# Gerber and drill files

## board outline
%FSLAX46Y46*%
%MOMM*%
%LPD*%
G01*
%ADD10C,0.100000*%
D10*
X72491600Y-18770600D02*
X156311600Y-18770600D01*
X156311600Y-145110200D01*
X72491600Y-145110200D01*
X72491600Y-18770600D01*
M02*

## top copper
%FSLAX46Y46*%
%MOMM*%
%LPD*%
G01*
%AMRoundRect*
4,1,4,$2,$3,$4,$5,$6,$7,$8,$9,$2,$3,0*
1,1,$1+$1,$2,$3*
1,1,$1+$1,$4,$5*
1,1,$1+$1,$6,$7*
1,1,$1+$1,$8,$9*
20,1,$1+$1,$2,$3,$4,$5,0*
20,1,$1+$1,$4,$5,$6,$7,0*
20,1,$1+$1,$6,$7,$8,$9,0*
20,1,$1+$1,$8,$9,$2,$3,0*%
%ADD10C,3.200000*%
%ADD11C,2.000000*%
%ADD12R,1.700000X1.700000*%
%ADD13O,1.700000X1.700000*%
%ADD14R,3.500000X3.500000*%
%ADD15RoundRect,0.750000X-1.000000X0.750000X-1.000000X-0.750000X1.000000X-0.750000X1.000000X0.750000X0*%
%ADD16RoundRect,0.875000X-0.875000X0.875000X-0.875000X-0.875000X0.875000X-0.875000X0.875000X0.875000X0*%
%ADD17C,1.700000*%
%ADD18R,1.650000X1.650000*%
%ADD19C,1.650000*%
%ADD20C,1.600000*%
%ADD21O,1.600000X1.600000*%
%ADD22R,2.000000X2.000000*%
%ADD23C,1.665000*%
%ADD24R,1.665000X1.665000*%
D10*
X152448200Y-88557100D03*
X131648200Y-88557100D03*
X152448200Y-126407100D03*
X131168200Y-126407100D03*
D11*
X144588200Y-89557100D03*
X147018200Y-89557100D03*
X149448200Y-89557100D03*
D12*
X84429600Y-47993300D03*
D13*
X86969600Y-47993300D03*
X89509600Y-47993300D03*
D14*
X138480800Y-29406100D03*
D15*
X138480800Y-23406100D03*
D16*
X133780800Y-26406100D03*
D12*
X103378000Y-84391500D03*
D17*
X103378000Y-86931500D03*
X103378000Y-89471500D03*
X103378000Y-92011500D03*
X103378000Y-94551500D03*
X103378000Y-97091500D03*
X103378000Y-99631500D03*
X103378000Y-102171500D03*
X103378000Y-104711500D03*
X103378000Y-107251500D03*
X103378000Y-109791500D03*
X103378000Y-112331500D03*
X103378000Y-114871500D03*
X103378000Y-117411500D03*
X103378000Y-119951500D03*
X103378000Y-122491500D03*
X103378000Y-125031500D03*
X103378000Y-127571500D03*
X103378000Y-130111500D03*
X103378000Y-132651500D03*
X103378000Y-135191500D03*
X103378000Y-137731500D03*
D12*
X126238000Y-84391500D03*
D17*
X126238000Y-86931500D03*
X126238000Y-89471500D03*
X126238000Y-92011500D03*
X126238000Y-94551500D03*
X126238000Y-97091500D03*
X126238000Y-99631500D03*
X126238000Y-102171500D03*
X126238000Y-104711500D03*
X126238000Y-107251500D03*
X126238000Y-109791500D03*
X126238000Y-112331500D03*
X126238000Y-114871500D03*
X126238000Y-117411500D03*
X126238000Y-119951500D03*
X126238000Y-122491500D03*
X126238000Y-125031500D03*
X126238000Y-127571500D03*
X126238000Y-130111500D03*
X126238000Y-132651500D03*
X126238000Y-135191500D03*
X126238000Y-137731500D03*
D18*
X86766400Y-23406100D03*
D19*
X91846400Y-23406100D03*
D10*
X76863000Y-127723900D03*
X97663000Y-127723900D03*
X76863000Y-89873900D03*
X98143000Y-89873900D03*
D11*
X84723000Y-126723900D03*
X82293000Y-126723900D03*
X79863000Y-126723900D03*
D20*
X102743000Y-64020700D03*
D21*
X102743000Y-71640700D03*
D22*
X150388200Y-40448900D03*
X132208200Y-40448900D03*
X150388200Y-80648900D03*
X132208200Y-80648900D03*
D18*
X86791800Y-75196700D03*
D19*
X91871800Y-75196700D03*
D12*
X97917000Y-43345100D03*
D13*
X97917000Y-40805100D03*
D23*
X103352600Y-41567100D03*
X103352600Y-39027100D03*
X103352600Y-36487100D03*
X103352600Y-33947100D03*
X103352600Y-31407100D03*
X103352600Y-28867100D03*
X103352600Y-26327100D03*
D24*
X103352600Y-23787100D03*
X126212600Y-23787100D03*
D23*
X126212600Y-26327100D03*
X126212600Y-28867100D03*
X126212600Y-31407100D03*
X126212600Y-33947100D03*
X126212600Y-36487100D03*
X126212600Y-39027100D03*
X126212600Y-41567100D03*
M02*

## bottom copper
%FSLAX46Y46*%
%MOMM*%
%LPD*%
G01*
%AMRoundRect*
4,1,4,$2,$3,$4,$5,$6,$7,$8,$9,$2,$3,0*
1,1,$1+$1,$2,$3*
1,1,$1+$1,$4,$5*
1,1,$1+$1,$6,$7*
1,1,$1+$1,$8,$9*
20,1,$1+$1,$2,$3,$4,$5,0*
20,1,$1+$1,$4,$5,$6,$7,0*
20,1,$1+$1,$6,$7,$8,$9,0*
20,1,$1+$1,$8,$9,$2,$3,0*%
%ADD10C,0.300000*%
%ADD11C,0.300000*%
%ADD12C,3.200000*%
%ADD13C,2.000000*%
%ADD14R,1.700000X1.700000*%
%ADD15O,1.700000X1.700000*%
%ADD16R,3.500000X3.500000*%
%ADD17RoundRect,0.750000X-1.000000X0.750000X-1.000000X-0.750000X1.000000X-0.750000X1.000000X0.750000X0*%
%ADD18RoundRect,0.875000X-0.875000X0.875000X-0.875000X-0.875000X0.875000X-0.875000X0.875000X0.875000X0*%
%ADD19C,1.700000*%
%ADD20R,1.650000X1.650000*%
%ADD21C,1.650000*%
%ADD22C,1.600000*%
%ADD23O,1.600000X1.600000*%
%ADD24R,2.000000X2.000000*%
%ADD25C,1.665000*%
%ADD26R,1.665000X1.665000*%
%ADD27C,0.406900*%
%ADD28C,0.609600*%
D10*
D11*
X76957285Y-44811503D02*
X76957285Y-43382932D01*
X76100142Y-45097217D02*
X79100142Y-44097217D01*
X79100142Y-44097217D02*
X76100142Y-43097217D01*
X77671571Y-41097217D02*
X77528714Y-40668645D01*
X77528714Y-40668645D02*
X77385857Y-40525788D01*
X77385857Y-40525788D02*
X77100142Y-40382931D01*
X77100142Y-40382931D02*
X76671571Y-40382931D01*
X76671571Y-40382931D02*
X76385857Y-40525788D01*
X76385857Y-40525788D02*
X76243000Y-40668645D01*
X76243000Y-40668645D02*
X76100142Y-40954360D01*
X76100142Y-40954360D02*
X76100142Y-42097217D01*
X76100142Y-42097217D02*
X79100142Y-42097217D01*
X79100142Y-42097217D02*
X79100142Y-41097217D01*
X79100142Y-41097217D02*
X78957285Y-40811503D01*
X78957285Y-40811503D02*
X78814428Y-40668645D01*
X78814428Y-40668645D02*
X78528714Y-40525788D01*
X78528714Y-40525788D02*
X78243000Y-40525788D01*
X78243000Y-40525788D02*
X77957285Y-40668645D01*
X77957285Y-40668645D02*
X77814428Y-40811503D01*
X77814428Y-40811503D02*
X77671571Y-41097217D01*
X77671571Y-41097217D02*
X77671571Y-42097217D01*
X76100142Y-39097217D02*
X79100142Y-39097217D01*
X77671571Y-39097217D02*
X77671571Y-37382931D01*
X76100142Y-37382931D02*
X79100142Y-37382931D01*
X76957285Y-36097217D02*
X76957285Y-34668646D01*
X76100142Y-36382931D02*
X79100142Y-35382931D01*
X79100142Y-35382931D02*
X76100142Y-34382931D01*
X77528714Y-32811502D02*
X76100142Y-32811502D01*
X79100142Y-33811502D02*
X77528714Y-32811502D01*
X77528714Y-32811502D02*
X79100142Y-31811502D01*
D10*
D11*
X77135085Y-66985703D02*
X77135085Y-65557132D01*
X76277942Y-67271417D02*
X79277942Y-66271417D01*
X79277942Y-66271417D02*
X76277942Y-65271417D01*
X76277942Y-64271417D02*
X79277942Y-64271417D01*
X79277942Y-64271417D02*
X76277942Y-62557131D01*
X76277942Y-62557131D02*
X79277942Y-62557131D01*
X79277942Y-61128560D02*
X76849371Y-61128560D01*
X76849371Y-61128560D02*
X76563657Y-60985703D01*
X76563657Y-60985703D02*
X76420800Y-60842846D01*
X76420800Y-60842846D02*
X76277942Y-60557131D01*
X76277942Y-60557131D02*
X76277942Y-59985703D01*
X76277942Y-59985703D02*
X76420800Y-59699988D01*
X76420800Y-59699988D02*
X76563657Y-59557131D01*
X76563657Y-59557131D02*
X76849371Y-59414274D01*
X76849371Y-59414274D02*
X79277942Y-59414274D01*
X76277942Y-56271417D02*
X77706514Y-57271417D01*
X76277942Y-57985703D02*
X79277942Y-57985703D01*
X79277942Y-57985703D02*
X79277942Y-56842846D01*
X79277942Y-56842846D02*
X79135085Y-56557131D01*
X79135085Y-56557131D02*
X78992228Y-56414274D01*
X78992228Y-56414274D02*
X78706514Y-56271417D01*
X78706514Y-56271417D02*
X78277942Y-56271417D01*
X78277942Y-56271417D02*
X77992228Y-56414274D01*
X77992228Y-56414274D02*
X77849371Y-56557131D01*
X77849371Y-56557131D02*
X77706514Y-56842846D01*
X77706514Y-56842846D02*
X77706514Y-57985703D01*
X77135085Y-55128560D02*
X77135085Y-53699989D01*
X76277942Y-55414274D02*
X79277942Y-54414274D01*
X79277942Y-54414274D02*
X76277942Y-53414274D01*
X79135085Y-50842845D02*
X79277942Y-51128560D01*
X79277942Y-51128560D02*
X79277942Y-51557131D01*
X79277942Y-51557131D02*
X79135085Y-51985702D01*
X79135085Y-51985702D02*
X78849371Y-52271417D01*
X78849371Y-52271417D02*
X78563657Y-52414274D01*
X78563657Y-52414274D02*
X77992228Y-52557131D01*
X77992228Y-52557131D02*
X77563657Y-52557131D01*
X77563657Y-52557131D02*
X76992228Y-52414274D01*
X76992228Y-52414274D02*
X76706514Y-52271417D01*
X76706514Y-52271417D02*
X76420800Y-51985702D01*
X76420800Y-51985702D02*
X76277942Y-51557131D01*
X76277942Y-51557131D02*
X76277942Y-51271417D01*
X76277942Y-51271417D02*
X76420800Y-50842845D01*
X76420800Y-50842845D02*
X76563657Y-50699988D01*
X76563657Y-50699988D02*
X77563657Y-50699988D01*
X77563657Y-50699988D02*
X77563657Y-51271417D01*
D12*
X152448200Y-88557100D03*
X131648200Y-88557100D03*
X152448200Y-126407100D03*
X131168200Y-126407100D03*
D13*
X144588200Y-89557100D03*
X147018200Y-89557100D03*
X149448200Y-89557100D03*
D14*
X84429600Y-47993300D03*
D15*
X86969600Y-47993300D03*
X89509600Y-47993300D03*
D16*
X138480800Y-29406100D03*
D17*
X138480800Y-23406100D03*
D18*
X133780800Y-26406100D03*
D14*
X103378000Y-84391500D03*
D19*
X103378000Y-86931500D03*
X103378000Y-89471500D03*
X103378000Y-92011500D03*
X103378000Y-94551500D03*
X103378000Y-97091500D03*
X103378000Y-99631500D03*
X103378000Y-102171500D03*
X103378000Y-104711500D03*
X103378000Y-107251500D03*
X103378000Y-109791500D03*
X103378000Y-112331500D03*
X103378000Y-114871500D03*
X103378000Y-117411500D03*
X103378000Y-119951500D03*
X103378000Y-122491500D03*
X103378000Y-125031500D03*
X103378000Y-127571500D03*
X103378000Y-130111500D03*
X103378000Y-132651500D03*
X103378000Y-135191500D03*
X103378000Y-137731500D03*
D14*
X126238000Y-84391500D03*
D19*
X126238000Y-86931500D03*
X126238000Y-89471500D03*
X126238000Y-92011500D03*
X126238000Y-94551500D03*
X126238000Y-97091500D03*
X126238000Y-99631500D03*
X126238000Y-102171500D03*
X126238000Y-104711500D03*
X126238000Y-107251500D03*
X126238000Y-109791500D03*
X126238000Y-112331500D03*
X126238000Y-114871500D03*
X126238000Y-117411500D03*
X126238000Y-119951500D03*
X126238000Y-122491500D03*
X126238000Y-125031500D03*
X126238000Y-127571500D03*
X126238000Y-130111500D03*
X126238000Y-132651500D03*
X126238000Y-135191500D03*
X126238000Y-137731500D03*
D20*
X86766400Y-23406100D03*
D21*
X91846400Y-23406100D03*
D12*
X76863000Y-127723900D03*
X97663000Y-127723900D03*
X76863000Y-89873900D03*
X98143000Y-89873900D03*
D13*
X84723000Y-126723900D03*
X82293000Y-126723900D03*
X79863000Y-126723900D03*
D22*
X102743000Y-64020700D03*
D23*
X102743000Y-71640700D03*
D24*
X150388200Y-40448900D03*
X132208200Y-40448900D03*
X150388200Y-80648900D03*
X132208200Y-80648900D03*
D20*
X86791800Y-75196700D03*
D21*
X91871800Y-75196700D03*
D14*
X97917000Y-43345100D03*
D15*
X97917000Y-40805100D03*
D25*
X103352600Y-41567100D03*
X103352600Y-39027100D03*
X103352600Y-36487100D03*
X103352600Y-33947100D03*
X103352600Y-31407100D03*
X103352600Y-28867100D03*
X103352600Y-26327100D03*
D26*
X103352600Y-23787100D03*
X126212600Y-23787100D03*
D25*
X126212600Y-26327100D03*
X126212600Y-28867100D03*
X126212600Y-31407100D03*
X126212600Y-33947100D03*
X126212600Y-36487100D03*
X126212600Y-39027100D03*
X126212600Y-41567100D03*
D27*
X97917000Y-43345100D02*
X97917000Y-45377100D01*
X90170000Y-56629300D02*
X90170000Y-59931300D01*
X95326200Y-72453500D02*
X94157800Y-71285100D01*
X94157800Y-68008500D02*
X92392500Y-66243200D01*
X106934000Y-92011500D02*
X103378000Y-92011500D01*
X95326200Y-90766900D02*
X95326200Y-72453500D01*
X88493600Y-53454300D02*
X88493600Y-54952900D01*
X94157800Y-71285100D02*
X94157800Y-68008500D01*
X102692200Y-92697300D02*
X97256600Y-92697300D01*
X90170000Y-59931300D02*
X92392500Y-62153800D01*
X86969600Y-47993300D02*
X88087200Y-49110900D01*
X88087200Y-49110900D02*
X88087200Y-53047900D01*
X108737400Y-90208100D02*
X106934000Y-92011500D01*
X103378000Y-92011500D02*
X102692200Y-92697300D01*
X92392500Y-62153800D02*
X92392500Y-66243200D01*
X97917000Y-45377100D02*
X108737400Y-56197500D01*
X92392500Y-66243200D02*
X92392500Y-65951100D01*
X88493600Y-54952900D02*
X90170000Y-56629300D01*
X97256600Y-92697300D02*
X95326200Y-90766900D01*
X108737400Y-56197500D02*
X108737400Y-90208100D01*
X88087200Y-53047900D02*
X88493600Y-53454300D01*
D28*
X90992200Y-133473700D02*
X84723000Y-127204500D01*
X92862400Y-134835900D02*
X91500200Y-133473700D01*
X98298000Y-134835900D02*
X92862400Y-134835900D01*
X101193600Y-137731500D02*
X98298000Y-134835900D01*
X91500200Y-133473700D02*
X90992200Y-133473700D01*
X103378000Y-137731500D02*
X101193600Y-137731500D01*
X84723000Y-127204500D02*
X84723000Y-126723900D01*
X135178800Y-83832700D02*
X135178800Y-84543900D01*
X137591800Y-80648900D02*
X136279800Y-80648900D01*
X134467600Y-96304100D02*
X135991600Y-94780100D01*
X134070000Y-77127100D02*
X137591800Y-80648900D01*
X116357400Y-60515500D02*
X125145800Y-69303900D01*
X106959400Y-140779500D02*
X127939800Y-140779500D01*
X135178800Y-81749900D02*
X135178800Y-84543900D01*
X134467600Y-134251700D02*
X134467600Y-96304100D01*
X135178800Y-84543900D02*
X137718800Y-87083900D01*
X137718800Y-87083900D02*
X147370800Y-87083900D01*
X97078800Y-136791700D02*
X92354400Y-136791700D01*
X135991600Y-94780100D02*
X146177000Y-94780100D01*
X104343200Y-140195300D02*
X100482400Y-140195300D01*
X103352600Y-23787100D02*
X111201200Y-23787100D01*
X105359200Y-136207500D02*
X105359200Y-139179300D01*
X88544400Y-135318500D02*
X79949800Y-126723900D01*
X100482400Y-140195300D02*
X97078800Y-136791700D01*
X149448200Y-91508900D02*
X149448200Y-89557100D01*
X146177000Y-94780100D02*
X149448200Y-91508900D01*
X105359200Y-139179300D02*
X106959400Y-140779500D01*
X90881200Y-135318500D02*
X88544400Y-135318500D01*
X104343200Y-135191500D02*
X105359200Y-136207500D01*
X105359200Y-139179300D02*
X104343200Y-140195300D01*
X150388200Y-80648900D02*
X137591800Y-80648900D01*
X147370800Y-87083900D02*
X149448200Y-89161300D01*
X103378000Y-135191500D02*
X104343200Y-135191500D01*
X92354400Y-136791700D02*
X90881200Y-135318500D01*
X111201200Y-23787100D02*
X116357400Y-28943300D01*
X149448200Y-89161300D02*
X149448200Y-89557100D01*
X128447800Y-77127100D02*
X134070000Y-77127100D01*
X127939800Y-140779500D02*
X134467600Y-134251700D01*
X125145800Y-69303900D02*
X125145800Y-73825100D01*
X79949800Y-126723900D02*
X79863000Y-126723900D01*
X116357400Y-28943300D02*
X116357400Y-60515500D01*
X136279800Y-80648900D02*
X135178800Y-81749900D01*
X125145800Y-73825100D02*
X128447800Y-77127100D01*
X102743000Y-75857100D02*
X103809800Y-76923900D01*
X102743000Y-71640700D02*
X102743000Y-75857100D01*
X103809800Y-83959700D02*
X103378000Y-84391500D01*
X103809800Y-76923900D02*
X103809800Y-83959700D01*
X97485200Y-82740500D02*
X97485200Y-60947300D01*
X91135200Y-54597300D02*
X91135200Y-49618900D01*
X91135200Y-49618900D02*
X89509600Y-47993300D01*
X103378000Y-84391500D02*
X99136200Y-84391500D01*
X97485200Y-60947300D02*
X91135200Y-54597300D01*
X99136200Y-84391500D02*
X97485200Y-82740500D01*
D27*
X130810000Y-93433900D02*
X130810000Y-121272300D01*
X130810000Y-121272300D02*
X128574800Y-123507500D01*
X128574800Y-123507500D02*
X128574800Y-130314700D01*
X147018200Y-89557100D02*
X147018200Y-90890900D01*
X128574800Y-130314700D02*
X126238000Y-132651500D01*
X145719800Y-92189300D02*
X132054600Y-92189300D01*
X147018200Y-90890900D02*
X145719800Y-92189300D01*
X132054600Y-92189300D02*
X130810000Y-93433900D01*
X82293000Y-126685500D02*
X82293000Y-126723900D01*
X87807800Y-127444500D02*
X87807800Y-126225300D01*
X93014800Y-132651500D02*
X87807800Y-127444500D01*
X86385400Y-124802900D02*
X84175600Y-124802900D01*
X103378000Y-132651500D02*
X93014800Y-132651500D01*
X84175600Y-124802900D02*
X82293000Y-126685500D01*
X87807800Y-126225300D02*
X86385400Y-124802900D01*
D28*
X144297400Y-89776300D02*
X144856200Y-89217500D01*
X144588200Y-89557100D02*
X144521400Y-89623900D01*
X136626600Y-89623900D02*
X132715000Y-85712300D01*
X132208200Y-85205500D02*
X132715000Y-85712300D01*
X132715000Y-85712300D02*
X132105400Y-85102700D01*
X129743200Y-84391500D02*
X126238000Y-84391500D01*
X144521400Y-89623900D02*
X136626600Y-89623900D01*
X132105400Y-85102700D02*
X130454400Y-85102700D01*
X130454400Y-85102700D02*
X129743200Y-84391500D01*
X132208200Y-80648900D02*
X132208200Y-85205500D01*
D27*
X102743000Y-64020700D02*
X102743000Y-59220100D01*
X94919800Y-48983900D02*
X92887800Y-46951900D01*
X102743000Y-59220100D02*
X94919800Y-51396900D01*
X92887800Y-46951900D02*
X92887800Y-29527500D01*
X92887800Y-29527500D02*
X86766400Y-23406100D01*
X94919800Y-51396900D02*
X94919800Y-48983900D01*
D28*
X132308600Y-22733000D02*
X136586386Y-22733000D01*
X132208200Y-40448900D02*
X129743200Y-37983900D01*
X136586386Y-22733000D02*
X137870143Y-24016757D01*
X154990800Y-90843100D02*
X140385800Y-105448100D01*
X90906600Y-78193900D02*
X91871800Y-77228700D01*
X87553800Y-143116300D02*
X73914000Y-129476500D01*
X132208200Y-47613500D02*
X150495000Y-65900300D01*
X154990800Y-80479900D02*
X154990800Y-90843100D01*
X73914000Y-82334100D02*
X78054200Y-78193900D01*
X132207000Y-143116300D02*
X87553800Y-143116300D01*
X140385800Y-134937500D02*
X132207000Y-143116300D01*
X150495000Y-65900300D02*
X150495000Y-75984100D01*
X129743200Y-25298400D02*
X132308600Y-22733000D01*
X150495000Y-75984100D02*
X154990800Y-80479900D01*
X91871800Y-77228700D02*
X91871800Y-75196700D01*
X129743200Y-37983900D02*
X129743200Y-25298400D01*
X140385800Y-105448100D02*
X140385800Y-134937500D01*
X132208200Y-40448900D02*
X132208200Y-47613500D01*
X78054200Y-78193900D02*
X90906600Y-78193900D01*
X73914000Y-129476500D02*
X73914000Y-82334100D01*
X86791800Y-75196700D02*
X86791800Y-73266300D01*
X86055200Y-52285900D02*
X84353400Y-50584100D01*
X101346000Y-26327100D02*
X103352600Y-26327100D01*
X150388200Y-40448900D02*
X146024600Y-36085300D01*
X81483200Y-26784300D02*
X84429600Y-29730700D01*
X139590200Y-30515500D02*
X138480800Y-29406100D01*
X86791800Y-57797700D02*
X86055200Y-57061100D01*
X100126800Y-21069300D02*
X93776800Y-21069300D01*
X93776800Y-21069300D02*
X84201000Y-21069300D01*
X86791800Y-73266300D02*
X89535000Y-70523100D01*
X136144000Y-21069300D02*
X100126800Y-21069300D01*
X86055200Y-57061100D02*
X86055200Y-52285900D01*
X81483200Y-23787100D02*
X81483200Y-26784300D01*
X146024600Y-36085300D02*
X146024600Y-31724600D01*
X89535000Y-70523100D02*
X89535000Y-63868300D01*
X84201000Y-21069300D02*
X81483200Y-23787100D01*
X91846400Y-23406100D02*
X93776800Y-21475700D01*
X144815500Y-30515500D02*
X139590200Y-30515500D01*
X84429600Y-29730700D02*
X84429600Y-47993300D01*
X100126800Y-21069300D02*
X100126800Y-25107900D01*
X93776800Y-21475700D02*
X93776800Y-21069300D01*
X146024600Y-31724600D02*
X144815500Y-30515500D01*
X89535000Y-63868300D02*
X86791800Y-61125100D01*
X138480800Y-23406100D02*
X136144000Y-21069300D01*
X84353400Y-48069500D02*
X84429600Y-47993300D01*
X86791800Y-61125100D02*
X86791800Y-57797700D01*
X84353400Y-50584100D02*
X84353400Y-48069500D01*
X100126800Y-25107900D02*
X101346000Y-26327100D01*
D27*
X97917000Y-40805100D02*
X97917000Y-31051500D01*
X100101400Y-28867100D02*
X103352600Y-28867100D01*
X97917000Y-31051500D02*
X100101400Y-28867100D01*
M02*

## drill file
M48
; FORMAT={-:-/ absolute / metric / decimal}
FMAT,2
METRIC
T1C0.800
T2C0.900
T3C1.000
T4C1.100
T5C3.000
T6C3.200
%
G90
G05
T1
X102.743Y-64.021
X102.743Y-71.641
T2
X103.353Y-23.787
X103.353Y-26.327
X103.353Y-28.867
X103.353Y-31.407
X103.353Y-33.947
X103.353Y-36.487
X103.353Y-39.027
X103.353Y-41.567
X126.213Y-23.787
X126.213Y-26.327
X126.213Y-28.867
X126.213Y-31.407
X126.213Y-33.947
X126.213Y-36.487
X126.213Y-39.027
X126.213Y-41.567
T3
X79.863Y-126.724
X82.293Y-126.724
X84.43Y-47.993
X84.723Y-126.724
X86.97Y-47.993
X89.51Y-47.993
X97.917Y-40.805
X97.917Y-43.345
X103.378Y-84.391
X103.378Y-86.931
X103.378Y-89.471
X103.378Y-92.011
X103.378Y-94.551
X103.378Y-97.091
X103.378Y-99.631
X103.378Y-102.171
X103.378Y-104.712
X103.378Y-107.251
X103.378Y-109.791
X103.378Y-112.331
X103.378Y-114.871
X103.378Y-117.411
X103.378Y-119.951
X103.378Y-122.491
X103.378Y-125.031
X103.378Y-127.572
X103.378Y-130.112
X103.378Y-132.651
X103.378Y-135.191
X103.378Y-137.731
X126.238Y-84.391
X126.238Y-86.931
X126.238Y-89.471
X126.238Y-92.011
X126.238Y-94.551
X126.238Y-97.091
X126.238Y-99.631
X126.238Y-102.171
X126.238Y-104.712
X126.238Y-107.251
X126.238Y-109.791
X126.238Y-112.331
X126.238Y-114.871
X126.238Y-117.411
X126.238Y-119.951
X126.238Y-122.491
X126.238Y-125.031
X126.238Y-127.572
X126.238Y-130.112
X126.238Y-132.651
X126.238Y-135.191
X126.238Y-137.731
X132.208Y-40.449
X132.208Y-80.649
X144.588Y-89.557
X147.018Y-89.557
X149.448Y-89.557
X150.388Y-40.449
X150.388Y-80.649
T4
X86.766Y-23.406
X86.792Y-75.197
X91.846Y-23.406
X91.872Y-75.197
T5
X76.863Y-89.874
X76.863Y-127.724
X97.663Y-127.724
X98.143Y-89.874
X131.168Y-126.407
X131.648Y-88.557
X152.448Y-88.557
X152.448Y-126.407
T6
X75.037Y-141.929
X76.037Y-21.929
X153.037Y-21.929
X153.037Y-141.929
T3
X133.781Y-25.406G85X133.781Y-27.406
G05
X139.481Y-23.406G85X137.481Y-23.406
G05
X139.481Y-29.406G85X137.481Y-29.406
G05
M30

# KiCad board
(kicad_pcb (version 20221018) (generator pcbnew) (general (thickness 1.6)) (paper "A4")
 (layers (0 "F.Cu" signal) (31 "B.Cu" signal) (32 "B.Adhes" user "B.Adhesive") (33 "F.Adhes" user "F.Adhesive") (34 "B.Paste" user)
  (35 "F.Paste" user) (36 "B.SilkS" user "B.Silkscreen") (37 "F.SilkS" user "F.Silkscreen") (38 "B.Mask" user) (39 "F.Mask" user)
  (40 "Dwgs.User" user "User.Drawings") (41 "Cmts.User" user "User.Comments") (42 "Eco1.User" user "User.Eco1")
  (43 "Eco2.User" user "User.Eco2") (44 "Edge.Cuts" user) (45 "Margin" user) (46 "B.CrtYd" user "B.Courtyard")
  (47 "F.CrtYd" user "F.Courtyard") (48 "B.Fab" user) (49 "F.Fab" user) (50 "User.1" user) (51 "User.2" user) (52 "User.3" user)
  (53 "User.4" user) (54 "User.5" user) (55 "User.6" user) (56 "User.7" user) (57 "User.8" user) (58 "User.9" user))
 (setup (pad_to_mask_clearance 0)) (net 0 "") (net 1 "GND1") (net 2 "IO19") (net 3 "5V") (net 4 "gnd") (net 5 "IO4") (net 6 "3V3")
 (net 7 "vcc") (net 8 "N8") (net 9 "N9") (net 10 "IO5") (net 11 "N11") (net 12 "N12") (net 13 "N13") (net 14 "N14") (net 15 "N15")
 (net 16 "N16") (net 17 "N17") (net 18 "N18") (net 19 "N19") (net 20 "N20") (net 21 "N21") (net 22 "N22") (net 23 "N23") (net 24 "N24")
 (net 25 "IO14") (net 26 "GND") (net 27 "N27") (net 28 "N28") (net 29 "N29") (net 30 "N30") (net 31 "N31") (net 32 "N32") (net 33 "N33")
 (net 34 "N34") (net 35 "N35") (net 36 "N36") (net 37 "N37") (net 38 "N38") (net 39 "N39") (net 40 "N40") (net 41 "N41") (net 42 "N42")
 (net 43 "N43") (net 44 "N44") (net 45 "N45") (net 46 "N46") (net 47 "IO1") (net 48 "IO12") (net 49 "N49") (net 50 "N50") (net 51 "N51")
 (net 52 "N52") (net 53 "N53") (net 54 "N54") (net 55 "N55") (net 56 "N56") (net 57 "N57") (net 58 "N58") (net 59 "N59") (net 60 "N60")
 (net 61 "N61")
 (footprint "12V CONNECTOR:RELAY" (layer "F.Cu") (at 131.6482 88.5571 -90)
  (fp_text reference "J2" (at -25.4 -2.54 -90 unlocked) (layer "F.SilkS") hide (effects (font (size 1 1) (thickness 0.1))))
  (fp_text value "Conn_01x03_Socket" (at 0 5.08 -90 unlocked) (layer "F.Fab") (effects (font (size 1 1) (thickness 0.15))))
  (pad "" np_thru_hole circle (at 0 -20.8 270) (size 3.2 3.2) (drill 3) (layers "F&B.Cu" "*.Mask"))
  (pad "" np_thru_hole circle (at 0 0 270) (size 3.2 3.2) (drill 3) (layers "F&B.Cu" "*.Mask"))
  (pad "" np_thru_hole circle (at 37.85 -20.8 270) (size 3.2 3.2) (drill 3) (layers "F&B.Cu" "*.Mask"))
  (pad "" np_thru_hole circle (at 37.85 0.48 270) (size 3.2 3.2) (drill 3) (layers "F&B.Cu" "*.Mask"))
  (pad "1" thru_hole circle (at 1 -12.94 270) (size 2 2) (drill 1) (layers "*.Cu" "*.Mask") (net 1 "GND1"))
  (pad "2" thru_hole circle (at 1 -15.37 270) (size 2 2) (drill 1) (layers "*.Cu" "*.Mask") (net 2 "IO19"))
  (pad "3" thru_hole circle (at 1 -17.8 270) (size 2 2) (drill 1) (layers "*.Cu" "*.Mask") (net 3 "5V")))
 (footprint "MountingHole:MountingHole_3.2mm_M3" (layer "F.Cu") (at 153.0368 21.9289)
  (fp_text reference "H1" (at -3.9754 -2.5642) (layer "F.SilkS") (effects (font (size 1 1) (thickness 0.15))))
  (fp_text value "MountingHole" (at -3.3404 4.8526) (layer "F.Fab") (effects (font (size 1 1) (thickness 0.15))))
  (pad "" np_thru_hole circle (at 0 0) (size 3.2 3.2) (drill 3.2) (layers "*.Cu" "*.Mask")))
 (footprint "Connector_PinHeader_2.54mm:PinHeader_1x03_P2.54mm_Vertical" (layer "F.Cu") (at 84.4296 47.9933 90)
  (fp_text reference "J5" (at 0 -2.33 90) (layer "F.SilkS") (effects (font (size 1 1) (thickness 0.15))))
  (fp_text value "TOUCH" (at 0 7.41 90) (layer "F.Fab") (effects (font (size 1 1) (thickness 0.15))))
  (pad "1" thru_hole rect (at 0 0 90) (size 1.7 1.7) (drill 1) (layers "*.Cu" "*.Mask") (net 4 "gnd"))
  (pad "2" thru_hole oval (at 0 2.54 90) (size 1.7 1.7) (drill 1) (layers "*.Cu" "*.Mask") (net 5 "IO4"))
  (pad "3" thru_hole oval (at 0 5.08 90) (size 1.7 1.7) (drill 1) (layers "*.Cu" "*.Mask") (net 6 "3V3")))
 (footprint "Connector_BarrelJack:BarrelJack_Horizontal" (layer "F.Cu") (at 138.4808 29.4061 -90)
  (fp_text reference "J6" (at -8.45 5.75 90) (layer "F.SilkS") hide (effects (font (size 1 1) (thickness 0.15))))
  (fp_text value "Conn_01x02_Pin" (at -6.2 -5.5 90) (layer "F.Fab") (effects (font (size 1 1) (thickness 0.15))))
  (pad "1" thru_hole rect (at 0 0 270) (size 3.5 3.5) (drill oval 1 3) (layers "*.Cu" "*.Mask") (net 4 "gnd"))
  (pad "2" thru_hole roundrect (at -6 0 270) (size 3 3.5) (drill oval 1 3) (layers "*.Cu" "*.Mask") (roundrect_rratio 0.25) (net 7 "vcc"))
  (pad "3" thru_hole roundrect (at -3 4.7 270) (size 3.5 3.5) (drill oval 3 1) (layers "*.Cu" "*.Mask") (roundrect_rratio 0.25)))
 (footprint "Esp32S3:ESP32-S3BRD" (layer "F.Cu") (at 102.108 149.1915)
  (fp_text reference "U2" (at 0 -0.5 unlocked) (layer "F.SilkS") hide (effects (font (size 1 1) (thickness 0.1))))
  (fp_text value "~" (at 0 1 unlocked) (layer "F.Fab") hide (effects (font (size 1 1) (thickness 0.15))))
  (pad "1_1" thru_hole rect (at 1.27 -64.8) (size 1.7 1.7) (drill 1) (layers "*.Cu" "*.Mask") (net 6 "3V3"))
  (pad "1_2" thru_hole circle (at 1.27 -62.26) (size 1.7 1.7) (drill 1) (layers "*.Cu" "*.Mask") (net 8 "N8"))
  (pad "1_3" thru_hole circle (at 1.27 -59.72) (size 1.7 1.7) (drill 1) (layers "*.Cu" "*.Mask") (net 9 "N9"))
  (pad "1_4" thru_hole circle (at 1.27 -57.18) (size 1.7 1.7) (drill 1) (layers "*.Cu" "*.Mask") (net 5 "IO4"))
  (pad "1_5" thru_hole circle (at 1.27 -54.64) (size 1.7 1.7) (drill 1) (layers "*.Cu" "*.Mask") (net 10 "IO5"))
  (pad "1_6" thru_hole circle (at 1.27 -52.1) (size 1.7 1.7) (drill 1) (layers "*.Cu" "*.Mask") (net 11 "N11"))
  (pad "1_7" thru_hole circle (at 1.27 -49.56) (size 1.7 1.7) (drill 1) (layers "*.Cu" "*.Mask") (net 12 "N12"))
  (pad "1_8" thru_hole circle (at 1.27 -47.02) (size 1.7 1.7) (drill 1) (layers "*.Cu" "*.Mask") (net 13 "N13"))
  (pad "1_9" thru_hole circle (at 1.27 -44.48) (size 1.7 1.7) (drill 1) (layers "*.Cu" "*.Mask") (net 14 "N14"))
  (pad "1_10" thru_hole circle (at 1.27 -41.94) (size 1.7 1.7) (drill 1) (layers "*.Cu" "*.Mask") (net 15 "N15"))
  (pad "1_11" thru_hole circle (at 1.27 -39.4) (size 1.7 1.7) (drill 1) (layers "*.Cu" "*.Mask") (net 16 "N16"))
  (pad "1_12" thru_hole circle (at 1.27 -36.86) (size 1.7 1.7) (drill 1) (layers "*.Cu" "*.Mask") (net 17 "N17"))
  (pad "1_13" thru_hole circle (at 1.27 -34.32) (size 1.7 1.7) (drill 1) (layers "*.Cu" "*.Mask") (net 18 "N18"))
  (pad "1_14" thru_hole circle (at 1.27 -31.78) (size 1.7 1.7) (drill 1) (layers "*.Cu" "*.Mask") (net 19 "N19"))
  (pad "1_15" thru_hole circle (at 1.27 -29.24) (size 1.7 1.7) (drill 1) (layers "*.Cu" "*.Mask") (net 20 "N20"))
  (pad "1_16" thru_hole circle (at 1.27 -26.7) (size 1.7 1.7) (drill 1) (layers "*.Cu" "*.Mask") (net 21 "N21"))
  (pad "1_17" thru_hole circle (at 1.27 -24.16) (size 1.7 1.7) (drill 1) (layers "*.Cu" "*.Mask") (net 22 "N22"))
  (pad "1_18" thru_hole circle (at 1.27 -21.62) (size 1.7 1.7) (drill 1) (layers "*.Cu" "*.Mask") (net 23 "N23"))
  (pad "1_19" thru_hole circle (at 1.27 -19.08) (size 1.7 1.7) (drill 1) (layers "*.Cu" "*.Mask") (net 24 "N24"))
  (pad "1_20" thru_hole circle (at 1.27 -16.54) (size 1.7 1.7) (drill 1) (layers "*.Cu" "*.Mask") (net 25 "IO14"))
  (pad "1_21" thru_hole circle (at 1.27 -14) (size 1.7 1.7) (drill 1) (layers "*.Cu" "*.Mask") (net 3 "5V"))
  (pad "1_22" thru_hole circle (at 1.27 -11.46) (size 1.7 1.7) (drill 1) (layers "*.Cu" "*.Mask") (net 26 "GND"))
  (pad "2_1" thru_hole rect (at 24.13 -64.8) (size 1.7 1.7) (drill 1) (layers "*.Cu" "*.Mask") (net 1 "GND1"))
  (pad "2_2" thru_hole circle (at 24.13 -62.26) (size 1.7 1.7) (drill 1) (layers "*.Cu" "*.Mask") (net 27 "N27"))
  (pad "2_3" thru_hole circle (at 24.13 -59.72) (size 1.7 1.7) (drill 1) (layers "*.Cu" "*.Mask") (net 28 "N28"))
  (pad "2_4" thru_hole circle (at 24.13 -57.18) (size 1.7 1.7) (drill 1) (layers "*.Cu" "*.Mask") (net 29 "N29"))
  (pad "2_5" thru_hole circle (at 24.13 -54.64) (size 1.7 1.7) (drill 1) (layers "*.Cu" "*.Mask") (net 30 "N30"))
  (pad "2_6" thru_hole circle (at 24.13 -52.1) (size 1.7 1.7) (drill 1) (layers "*.Cu" "*.Mask") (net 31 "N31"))
  (pad "2_7" thru_hole circle (at 24.13 -49.56) (size 1.7 1.7) (drill 1) (layers "*.Cu" "*.Mask") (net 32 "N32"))
  (pad "2_8" thru_hole circle (at 24.13 -47.02) (size 1.7 1.7) (drill 1) (layers "*.Cu" "*.Mask") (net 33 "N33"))
  (pad "2_9" thru_hole circle (at 24.13 -44.48) (size 1.7 1.7) (drill 1) (layers "*.Cu" "*.Mask") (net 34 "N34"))
  (pad "2_10" thru_hole circle (at 24.13 -41.94) (size 1.7 1.7) (drill 1) (layers "*.Cu" "*.Mask") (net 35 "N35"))
  (pad "2_11" thru_hole circle (at 24.13 -39.4) (size 1.7 1.7) (drill 1) (layers "*.Cu" "*.Mask") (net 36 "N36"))
  (pad "2_12" thru_hole circle (at 24.13 -36.86) (size 1.7 1.7) (drill 1) (layers "*.Cu" "*.Mask") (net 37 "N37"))
  (pad "2_13" thru_hole circle (at 24.13 -34.32) (size 1.7 1.7) (drill 1) (layers "*.Cu" "*.Mask") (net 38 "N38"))
  (pad "2_14" thru_hole circle (at 24.13 -31.78) (size 1.7 1.7) (drill 1) (layers "*.Cu" "*.Mask") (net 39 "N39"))
  (pad "2_15" thru_hole circle (at 24.13 -29.24) (size 1.7 1.7) (drill 1) (layers "*.Cu" "*.Mask") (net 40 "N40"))
  (pad "2_16" thru_hole circle (at 24.13 -26.7) (size 1.7 1.7) (drill 1) (layers "*.Cu" "*.Mask") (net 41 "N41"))
  (pad "2_17" thru_hole circle (at 24.13 -24.16) (size 1.7 1.7) (drill 1) (layers "*.Cu" "*.Mask") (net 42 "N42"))
  (pad "2_18" thru_hole circle (at 24.13 -21.62) (size 1.7 1.7) (drill 1) (layers "*.Cu" "*.Mask") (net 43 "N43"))
  (pad "2_19" thru_hole circle (at 24.13 -19.08) (size 1.7 1.7) (drill 1) (layers "*.Cu" "*.Mask") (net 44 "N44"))
  (pad "2_20" thru_hole circle (at 24.13 -16.54) (size 1.7 1.7) (drill 1) (layers "*.Cu" "*.Mask") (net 2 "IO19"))
  (pad "2_21" thru_hole circle (at 24.13 -14) (size 1.7 1.7) (drill 1) (layers "*.Cu" "*.Mask") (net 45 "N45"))
  (pad "2_22" thru_hole circle (at 24.13 -11.46) (size 1.7 1.7) (drill 1) (layers "*.Cu" "*.Mask") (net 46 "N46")))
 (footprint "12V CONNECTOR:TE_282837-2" (layer "F.Cu") (at 89.3064 23.4061)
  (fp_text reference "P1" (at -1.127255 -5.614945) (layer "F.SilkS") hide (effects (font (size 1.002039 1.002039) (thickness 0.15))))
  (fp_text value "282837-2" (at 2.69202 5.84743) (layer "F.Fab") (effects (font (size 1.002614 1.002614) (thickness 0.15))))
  (pad "1" thru_hole rect (at -2.54 0) (size 1.65 1.65) (drill 1.1) (layers "*.Cu" "*.Mask") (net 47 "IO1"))
  (pad "2" thru_hole circle (at 2.54 0) (size 1.65 1.65) (drill 1.1) (layers "*.Cu" "*.Mask") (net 4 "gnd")))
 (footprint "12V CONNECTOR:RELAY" (layer "F.Cu") (at 97.663 127.7239 90)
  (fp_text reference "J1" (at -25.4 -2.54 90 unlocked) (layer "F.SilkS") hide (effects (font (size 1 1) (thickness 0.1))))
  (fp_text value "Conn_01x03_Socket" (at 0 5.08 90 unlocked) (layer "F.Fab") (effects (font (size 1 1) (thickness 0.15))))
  (pad "" np_thru_hole circle (at 0 -20.8 90) (size 3.2 3.2) (drill 3) (layers "F&B.Cu" "*.Mask"))
  (pad "" np_thru_hole circle (at 0 0 90) (size 3.2 3.2) (drill 3) (layers "F&B.Cu" "*.Mask"))
  (pad "" np_thru_hole circle (at 37.85 -20.8 90) (size 3.2 3.2) (drill 3) (layers "F&B.Cu" "*.Mask"))
  (pad "" np_thru_hole circle (at 37.85 0.48 90) (size 3.2 3.2) (drill 3) (layers "F&B.Cu" "*.Mask"))
  (pad "1" thru_hole circle (at 1 -12.94 90) (size 2 2) (drill 1) (layers "*.Cu" "*.Mask") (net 26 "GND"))
  (pad "2" thru_hole circle (at 1 -15.37 90) (size 2 2) (drill 1) (layers "*.Cu" "*.Mask") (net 25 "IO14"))
  (pad "3" thru_hole circle (at 1 -17.8 90) (size 2 2) (drill 1) (layers "*.Cu" "*.Mask") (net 3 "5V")))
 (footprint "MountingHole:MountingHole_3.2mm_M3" (layer "F.Cu") (at 153.0368 141.9289)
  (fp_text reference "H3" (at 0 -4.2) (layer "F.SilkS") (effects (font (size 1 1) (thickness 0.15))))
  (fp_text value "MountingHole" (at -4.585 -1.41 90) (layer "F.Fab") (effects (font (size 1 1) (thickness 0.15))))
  (pad "" np_thru_hole circle (at 0 0) (size 3.2 3.2) (drill 3.2) (layers "*.Cu" "*.Mask")))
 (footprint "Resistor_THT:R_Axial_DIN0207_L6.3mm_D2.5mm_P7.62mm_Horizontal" (layer "F.Cu") (at 102.743 64.0207 -90)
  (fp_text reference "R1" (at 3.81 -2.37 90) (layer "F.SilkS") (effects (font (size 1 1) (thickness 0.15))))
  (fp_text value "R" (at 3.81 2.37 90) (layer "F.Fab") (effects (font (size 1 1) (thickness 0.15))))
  (pad "1" thru_hole circle (at 0 0 270) (size 1.6 1.6) (drill 0.8) (layers "*.Cu" "*.Mask") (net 47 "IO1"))
  (pad "2" thru_hole oval (at 7.62 0 270) (size 1.6 1.6) (drill 0.8) (layers "*.Cu" "*.Mask") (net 6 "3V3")))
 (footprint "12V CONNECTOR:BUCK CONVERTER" (layer "F.Cu") (at 130.4082 38.6489 -90)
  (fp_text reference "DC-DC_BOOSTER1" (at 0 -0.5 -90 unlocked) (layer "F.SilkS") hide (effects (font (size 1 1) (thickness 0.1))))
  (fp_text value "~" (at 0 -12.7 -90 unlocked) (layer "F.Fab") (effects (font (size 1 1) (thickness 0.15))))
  (pad "IN+" thru_hole rect (at 1.8 -19.98 270) (size 2 2) (drill 1) (layers "*.Cu" "*.Mask") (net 4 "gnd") (thermal_bridge_angle 45))
  (pad "IN-" thru_hole rect (at 1.8 -1.8 270) (size 2 2) (drill 1) (layers "*.Cu" "B.Mask") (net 7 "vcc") (thermal_bridge_angle 45))
  (pad "OUT+" thru_hole rect (at 42 -19.98 270) (size 2 2) (drill 1) (layers "*.Cu" "*.Mask") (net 3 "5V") (thermal_bridge_angle 45))
  (pad "OUT-" thru_hole rect (at 42 -1.8 270) (size 2 2) (drill 1) (layers "*.Cu" "*.Mask") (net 1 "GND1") (thermal_bridge_angle 45)))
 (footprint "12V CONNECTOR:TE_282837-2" (layer "F.Cu") (at 89.3318 75.1967)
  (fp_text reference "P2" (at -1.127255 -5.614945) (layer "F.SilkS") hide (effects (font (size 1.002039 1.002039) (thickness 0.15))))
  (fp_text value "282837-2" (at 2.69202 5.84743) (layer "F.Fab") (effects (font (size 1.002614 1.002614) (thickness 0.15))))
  (pad "1" thru_hole rect (at -2.54 0) (size 1.65 1.65) (drill 1.1) (layers "*.Cu" "*.Mask") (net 4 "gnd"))
  (pad "2" thru_hole circle (at 2.54 0) (size 1.65 1.65) (drill 1.1) (layers "*.Cu" "*.Mask") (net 7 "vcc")))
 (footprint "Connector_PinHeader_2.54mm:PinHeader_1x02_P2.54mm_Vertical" (layer "F.Cu") (at 97.917 43.3451 180)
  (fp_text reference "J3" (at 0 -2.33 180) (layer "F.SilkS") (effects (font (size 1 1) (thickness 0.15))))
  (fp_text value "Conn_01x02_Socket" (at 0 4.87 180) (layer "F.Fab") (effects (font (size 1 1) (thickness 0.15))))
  (pad "1" thru_hole rect (at 0 0 180) (size 1.7 1.7) (drill 1) (layers "*.Cu" "*.Mask") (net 5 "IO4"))
  (pad "2" thru_hole oval (at 0 2.54 180) (size 1.7 1.7) (drill 1) (layers "*.Cu" "*.Mask") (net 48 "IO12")))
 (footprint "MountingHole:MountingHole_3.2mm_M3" (layer "F.Cu") (at 75.0368 141.9289)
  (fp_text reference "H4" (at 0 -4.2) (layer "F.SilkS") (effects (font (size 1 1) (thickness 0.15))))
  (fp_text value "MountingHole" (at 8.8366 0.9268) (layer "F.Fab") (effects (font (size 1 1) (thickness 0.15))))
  (pad "" np_thru_hole circle (at 0 0) (size 3.2 3.2) (drill 3.2) (layers "*.Cu" "*.Mask")))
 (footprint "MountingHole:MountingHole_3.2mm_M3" (layer "F.Cu") (at 76.0368 21.9289)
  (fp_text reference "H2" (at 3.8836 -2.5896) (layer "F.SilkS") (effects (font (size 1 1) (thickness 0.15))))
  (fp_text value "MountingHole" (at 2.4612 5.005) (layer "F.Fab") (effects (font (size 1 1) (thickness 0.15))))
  (pad "" np_thru_hole circle (at 0 0) (size 3.2 3.2) (drill 3.2) (layers "*.Cu" "*.Mask")))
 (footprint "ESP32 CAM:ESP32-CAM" (layer "F.Cu") (at 103.3526 41.5671)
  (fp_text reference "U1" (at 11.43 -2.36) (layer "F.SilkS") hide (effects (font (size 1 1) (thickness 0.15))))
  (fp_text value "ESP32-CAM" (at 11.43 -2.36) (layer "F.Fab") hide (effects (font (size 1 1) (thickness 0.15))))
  (pad "1" thru_hole circle (at 0 0) (size 1.665 1.665) (drill 0.9) (layers "*.Cu" "*.Mask") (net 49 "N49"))
  (pad "2" thru_hole circle (at 0 -2.54) (size 1.665 1.665) (drill 0.9) (layers "*.Cu" "*.Mask") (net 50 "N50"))
  (pad "3" thru_hole circle (at 0 -5.08) (size 1.665 1.665) (drill 0.9) (layers "*.Cu" "*.Mask") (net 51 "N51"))
  (pad "4" thru_hole circle (at 0 -7.62) (size 1.665 1.665) (drill 0.9) (layers "*.Cu" "*.Mask") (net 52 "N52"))
  (pad "5" thru_hole circle (at 0 -10.16) (size 1.665 1.665) (drill 0.9) (layers "*.Cu" "*.Mask") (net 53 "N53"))
  (pad "6" thru_hole circle (at 0 -12.7) (size 1.665 1.665) (drill 0.9) (layers "*.Cu" "*.Mask") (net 48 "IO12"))
  (pad "7" thru_hole circle (at 0 -15.24) (size 1.665 1.665) (drill 0.9) (layers "*.Cu" "*.Mask") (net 4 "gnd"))
  (pad "8" thru_hole rect (at 0 -17.78) (size 1.665 1.665) (drill 0.9) (layers "*.Cu" "*.Mask") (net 3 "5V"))
  (pad "9" thru_hole rect (at 22.86 -17.78) (size 1.665 1.665) (drill 0.9) (layers "*.Cu" "*.Mask") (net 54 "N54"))
  (pad "10" thru_hole circle (at 22.86 -15.24) (size 1.665 1.665) (drill 0.9) (layers "*.Cu" "*.Mask") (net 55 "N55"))
  (pad "11" thru_hole circle (at 22.86 -12.7) (size 1.665 1.665) (drill 0.9) (layers "*.Cu" "*.Mask") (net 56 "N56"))
  (pad "12" thru_hole circle (at 22.86 -10.16) (size 1.665 1.665) (drill 0.9) (layers "*.Cu" "*.Mask") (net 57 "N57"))
  (pad "13" thru_hole circle (at 22.86 -7.62) (size 1.665 1.665) (drill 0.9) (layers "*.Cu" "*.Mask") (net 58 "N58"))
  (pad "14" thru_hole circle (at 22.86 -5.08) (size 1.665 1.665) (drill 0.9) (layers "*.Cu" "*.Mask") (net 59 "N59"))
  (pad "15" thru_hole circle (at 22.86 -2.54) (size 1.665 1.665) (drill 0.9) (layers "*.Cu" "*.Mask") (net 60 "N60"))
  (pad "16" thru_hole circle (at 22.86 0) (size 1.665 1.665) (drill 0.9) (layers "*.Cu" "*.Mask") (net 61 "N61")))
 (gr_rect (start 72.4916 18.7706) (end 156.3116 145.1102) (stroke (width 0.1) (type default)) (fill none) (layer "Edge.Cuts"))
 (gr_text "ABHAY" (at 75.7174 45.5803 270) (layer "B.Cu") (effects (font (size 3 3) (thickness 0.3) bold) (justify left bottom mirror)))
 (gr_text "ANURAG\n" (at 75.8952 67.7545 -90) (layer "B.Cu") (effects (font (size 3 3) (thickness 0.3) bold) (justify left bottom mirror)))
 (segment (start 97.917 43.3451) (end 97.917 45.3771) (width 0.4069) (layer "B.Cu") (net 5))
 (segment (start 90.17 56.6293) (end 90.17 59.9313) (width 0.4069) (layer "B.Cu") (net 5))
 (segment (start 95.3262 72.4535) (end 94.1578 71.2851) (width 0.4069) (layer "B.Cu") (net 5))
 (segment (start 94.1578 68.0085) (end 92.3925 66.2432) (width 0.4069) (layer "B.Cu") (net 5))
 (segment (start 106.934 92.0115) (end 103.378 92.0115) (width 0.4069) (layer "B.Cu") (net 5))
 (segment (start 95.3262 90.7669) (end 95.3262 72.4535) (width 0.4069) (layer "B.Cu") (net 5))
 (segment (start 88.4936 53.4543) (end 88.4936 54.9529) (width 0.4069) (layer "B.Cu") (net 5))
 (segment (start 94.1578 71.2851) (end 94.1578 68.0085) (width 0.4069) (layer "B.Cu") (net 5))
 (segment (start 102.6922 92.6973) (end 97.2566 92.6973) (width 0.4069) (layer "B.Cu") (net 5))
 (segment (start 90.17 59.9313) (end 92.3925 62.1538) (width 0.4069) (layer "B.Cu") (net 5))
 (segment (start 86.9696 47.9933) (end 88.0872 49.1109) (width 0.4069) (layer "B.Cu") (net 5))
 (segment (start 88.0872 49.1109) (end 88.0872 53.0479) (width 0.4069) (layer "B.Cu") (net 5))
 (segment (start 108.7374 90.2081) (end 106.934 92.0115) (width 0.4069) (layer "B.Cu") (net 5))
 (segment (start 103.378 92.0115) (end 102.6922 92.6973) (width 0.4069) (layer "B.Cu") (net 5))
 (segment (start 92.3925 62.1538) (end 92.3925 66.2432) (width 0.4069) (layer "B.Cu") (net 5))
 (segment (start 97.917 45.3771) (end 108.7374 56.1975) (width 0.4069) (layer "B.Cu") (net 5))
 (segment (start 92.3925 66.2432) (end 92.3925 65.9511) (width 0.4069) (layer "B.Cu") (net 5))
 (segment (start 88.4936 54.9529) (end 90.17 56.6293) (width 0.4069) (layer "B.Cu") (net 5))
 (segment (start 97.2566 92.6973) (end 95.3262 90.7669) (width 0.4069) (layer "B.Cu") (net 5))
 (segment (start 108.7374 56.1975) (end 108.7374 90.2081) (width 0.4069) (layer "B.Cu") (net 5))
 (segment (start 88.0872 53.0479) (end 88.4936 53.4543) (width 0.4069) (layer "B.Cu") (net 5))
 (segment (start 90.9922 133.4737) (end 84.723 127.2045) (width 0.6096) (layer "B.Cu") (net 26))
 (segment (start 92.8624 134.8359) (end 91.5002 133.4737) (width 0.6096) (layer "B.Cu") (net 26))
 (segment (start 98.298 134.8359) (end 92.8624 134.8359) (width 0.6096) (layer "B.Cu") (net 26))
 (segment (start 101.1936 137.7315) (end 98.298 134.8359) (width 0.6096) (layer "B.Cu") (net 26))
 (segment (start 91.5002 133.4737) (end 90.9922 133.4737) (width 0.6096) (layer "B.Cu") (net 26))
 (segment (start 103.378 137.7315) (end 101.1936 137.7315) (width 0.6096) (layer "B.Cu") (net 26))
 (segment (start 84.723 127.2045) (end 84.723 126.7239) (width 0.6096) (layer "B.Cu") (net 26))
 (segment (start 135.1788 83.8327) (end 135.1788 84.5439) (width 0.6096) (layer "B.Cu") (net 3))
 (segment (start 137.5918 80.6489) (end 136.2798 80.6489) (width 0.6096) (layer "B.Cu") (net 3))
 (segment (start 134.4676 96.3041) (end 135.9916 94.7801) (width 0.6096) (layer "B.Cu") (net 3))
 (segment (start 134.07 77.1271) (end 137.5918 80.6489) (width 0.6096) (layer "B.Cu") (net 3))
 (segment (start 116.3574 60.5155) (end 125.1458 69.3039) (width 0.6096) (layer "B.Cu") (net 3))
 (segment (start 106.9594 140.7795) (end 127.9398 140.7795) (width 0.6096) (layer "B.Cu") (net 3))
 (segment (start 135.1788 81.7499) (end 135.1788 84.5439) (width 0.6096) (layer "B.Cu") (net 3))
 (segment (start 134.4676 134.2517) (end 134.4676 96.3041) (width 0.6096) (layer "B.Cu") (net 3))
 (segment (start 135.1788 84.5439) (end 137.7188 87.0839) (width 0.6096) (layer "B.Cu") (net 3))
 (segment (start 137.7188 87.0839) (end 147.3708 87.0839) (width 0.6096) (layer "B.Cu") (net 3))
 (segment (start 97.0788 136.7917) (end 92.3544 136.7917) (width 0.6096) (layer "B.Cu") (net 3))
 (segment (start 135.9916 94.7801) (end 146.177 94.7801) (width 0.6096) (layer "B.Cu") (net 3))
 (segment (start 104.3432 140.1953) (end 100.4824 140.1953) (width 0.6096) (layer "B.Cu") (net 3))
 (segment (start 103.3526 23.7871) (end 111.2012 23.7871) (width 0.6096) (layer "B.Cu") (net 3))
 (segment (start 105.3592 136.2075) (end 105.3592 139.1793) (width 0.6096) (layer "B.Cu") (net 3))
 (segment (start 88.5444 135.3185) (end 79.9498 126.7239) (width 0.6096) (layer "B.Cu") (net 3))
 (segment (start 100.4824 140.1953) (end 97.0788 136.7917) (width 0.6096) (layer "B.Cu") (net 3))
 (segment (start 149.4482 91.5089) (end 149.4482 89.5571) (width 0.6096) (layer "B.Cu") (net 3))
 (segment (start 146.177 94.7801) (end 149.4482 91.5089) (width 0.6096) (layer "B.Cu") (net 3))
 (segment (start 105.3592 139.1793) (end 106.9594 140.7795) (width 0.6096) (layer "B.Cu") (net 3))
 (segment (start 90.8812 135.3185) (end 88.5444 135.3185) (width 0.6096) (layer "B.Cu") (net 3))
 (segment (start 104.3432 135.1915) (end 105.3592 136.2075) (width 0.6096) (layer "B.Cu") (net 3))
 (segment (start 105.3592 139.1793) (end 104.3432 140.1953) (width 0.6096) (layer "B.Cu") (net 3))
 (segment (start 150.3882 80.6489) (end 137.5918 80.6489) (width 0.6096) (layer "B.Cu") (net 3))
 (segment (start 147.3708 87.0839) (end 149.4482 89.1613) (width 0.6096) (layer "B.Cu") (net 3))
 (segment (start 103.378 135.1915) (end 104.3432 135.1915) (width 0.6096) (layer "B.Cu") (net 3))
 (segment (start 92.3544 136.7917) (end 90.8812 135.3185) (width 0.6096) (layer "B.Cu") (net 3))
 (segment (start 111.2012 23.7871) (end 116.3574 28.9433) (width 0.6096) (layer "B.Cu") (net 3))
 (segment (start 149.4482 89.1613) (end 149.4482 89.5571) (width 0.6096) (layer "B.Cu") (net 3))
 (segment (start 128.4478 77.1271) (end 134.07 77.1271) (width 0.6096) (layer "B.Cu") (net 3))
 (segment (start 127.9398 140.7795) (end 134.4676 134.2517) (width 0.6096) (layer "B.Cu") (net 3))
 (segment (start 125.1458 69.3039) (end 125.1458 73.8251) (width 0.6096) (layer "B.Cu") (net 3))
 (segment (start 79.9498 126.7239) (end 79.863 126.7239) (width 0.6096) (layer "B.Cu") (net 3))
 (segment (start 116.3574 28.9433) (end 116.3574 60.5155) (width 0.6096) (layer "B.Cu") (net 3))
 (segment (start 136.2798 80.6489) (end 135.1788 81.7499) (width 0.6096) (layer "B.Cu") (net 3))
 (segment (start 125.1458 73.8251) (end 128.4478 77.1271) (width 0.6096) (layer "B.Cu") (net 3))
 (segment (start 102.743 75.8571) (end 103.8098 76.9239) (width 0.6096) (layer "B.Cu") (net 6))
 (segment (start 102.743 71.6407) (end 102.743 75.8571) (width 0.6096) (layer "B.Cu") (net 6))
 (segment (start 103.8098 83.9597) (end 103.378 84.3915) (width 0.6096) (layer "B.Cu") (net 6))
 (segment (start 103.8098 76.9239) (end 103.8098 83.9597) (width 0.6096) (layer "B.Cu") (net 6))
 (segment (start 97.4852 82.7405) (end 97.4852 60.9473) (width 0.6096) (layer "B.Cu") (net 6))
 (segment (start 91.1352 54.5973) (end 91.1352 49.6189) (width 0.6096) (layer "B.Cu") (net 6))
 (segment (start 91.1352 49.6189) (end 89.5096 47.9933) (width 0.6096) (layer "B.Cu") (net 6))
 (segment (start 103.378 84.3915) (end 99.1362 84.3915) (width 0.6096) (layer "B.Cu") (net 6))
 (segment (start 97.4852 60.9473) (end 91.1352 54.5973) (width 0.6096) (layer "B.Cu") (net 6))
 (segment (start 99.1362 84.3915) (end 97.4852 82.7405) (width 0.6096) (layer "B.Cu") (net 6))
 (segment (start 130.81 93.4339) (end 130.81 121.2723) (width 0.4069) (layer "B.Cu") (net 2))
 (segment (start 130.81 121.2723) (end 128.5748 123.5075) (width 0.4069) (layer "B.Cu") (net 2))
 (segment (start 128.5748 123.5075) (end 128.5748 130.3147) (width 0.4069) (layer "B.Cu") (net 2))
 (segment (start 147.0182 89.5571) (end 147.0182 90.8909) (width 0.4069) (layer "B.Cu") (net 2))
 (segment (start 128.5748 130.3147) (end 126.238 132.6515) (width 0.4069) (layer "B.Cu") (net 2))
 (segment (start 145.7198 92.1893) (end 132.0546 92.1893) (width 0.4069) (layer "B.Cu") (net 2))
 (segment (start 147.0182 90.8909) (end 145.7198 92.1893) (width 0.4069) (layer "B.Cu") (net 2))
 (segment (start 132.0546 92.1893) (end 130.81 93.4339) (width 0.4069) (layer "B.Cu") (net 2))
 (segment (start 82.293 126.6855) (end 82.293 126.7239) (width 0.4069) (layer "B.Cu") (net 25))
 (segment (start 87.8078 127.4445) (end 87.8078 126.2253) (width 0.4069) (layer "B.Cu") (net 25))
 (segment (start 93.0148 132.6515) (end 87.8078 127.4445) (width 0.4069) (layer "B.Cu") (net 25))
 (segment (start 86.3854 124.8029) (end 84.1756 124.8029) (width 0.4069) (layer "B.Cu") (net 25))
 (segment (start 103.378 132.6515) (end 93.0148 132.6515) (width 0.4069) (layer "B.Cu") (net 25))
 (segment (start 84.1756 124.8029) (end 82.293 126.6855) (width 0.4069) (layer "B.Cu") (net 25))
 (segment (start 87.8078 126.2253) (end 86.3854 124.8029) (width 0.4069) (layer "B.Cu") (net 25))
 (segment (start 144.2974 89.7763) (end 144.8562 89.2175) (width 0.6096) (layer "B.Cu") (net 1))
 (segment (start 144.5882 89.5571) (end 144.5214 89.6239) (width 0.6096) (layer "B.Cu") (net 1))
 (segment (start 136.6266 89.6239) (end 132.715 85.7123) (width 0.6096) (layer "B.Cu") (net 1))
 (segment (start 132.2082 85.2055) (end 132.715 85.7123) (width 0.6096) (layer "B.Cu") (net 1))
 (segment (start 132.715 85.7123) (end 132.1054 85.1027) (width 0.6096) (layer "B.Cu") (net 1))
 (segment (start 129.7432 84.3915) (end 126.238 84.3915) (width 0.6096) (layer "B.Cu") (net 1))
 (segment (start 144.5214 89.6239) (end 136.6266 89.6239) (width 0.6096) (layer "B.Cu") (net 1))
 (segment (start 132.1054 85.1027) (end 130.4544 85.1027) (width 0.6096) (layer "B.Cu") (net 1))
 (segment (start 130.4544 85.1027) (end 129.7432 84.3915) (width 0.6096) (layer "B.Cu") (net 1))
 (segment (start 132.2082 80.6489) (end 132.2082 85.2055) (width 0.6096) (layer "B.Cu") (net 1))
 (segment (start 102.743 64.0207) (end 102.743 59.2201) (width 0.4069) (layer "B.Cu") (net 47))
 (segment (start 94.9198 48.9839) (end 92.8878 46.9519) (width 0.4069) (layer "B.Cu") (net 47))
 (segment (start 102.743 59.2201) (end 94.9198 51.3969) (width 0.4069) (layer "B.Cu") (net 47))
 (segment (start 92.8878 46.9519) (end 92.8878 29.5275) (width 0.4069) (layer "B.Cu") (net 47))
 (segment (start 92.8878 29.5275) (end 86.7664 23.4061) (width 0.4069) (layer "B.Cu") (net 47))
 (segment (start 94.9198 51.3969) (end 94.9198 48.9839) (width 0.4069) (layer "B.Cu") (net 47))
 (segment (start 132.3086 22.733) (end 136.586386 22.733) (width 0.6096) (layer "B.Cu") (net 7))
 (segment (start 132.2082 40.4489) (end 129.7432 37.9839) (width 0.6096) (layer "B.Cu") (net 7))
 (segment (start 136.586386 22.733) (end 137.870143 24.016757) (width 0.6096) (layer "B.Cu") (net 7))
 (segment (start 154.9908 90.8431) (end 140.3858 105.4481) (width 0.6096) (layer "B.Cu") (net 7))
 (segment (start 90.9066 78.1939) (end 91.8718 77.2287) (width 0.6096) (layer "B.Cu") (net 7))
 (segment (start 87.5538 143.1163) (end 73.914 129.4765) (width 0.6096) (layer "B.Cu") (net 7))
 (segment (start 132.2082 47.6135) (end 150.495 65.9003) (width 0.6096) (layer "B.Cu") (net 7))
 (segment (start 154.9908 80.4799) (end 154.9908 90.8431) (width 0.6096) (layer "B.Cu") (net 7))
 (segment (start 73.914 82.3341) (end 78.0542 78.1939) (width 0.6096) (layer "B.Cu") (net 7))
 (segment (start 132.207 143.1163) (end 87.5538 143.1163) (width 0.6096) (layer "B.Cu") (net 7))
 (segment (start 140.3858 134.9375) (end 132.207 143.1163) (width 0.6096) (layer "B.Cu") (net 7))
 (segment (start 150.495 65.9003) (end 150.495 75.9841) (width 0.6096) (layer "B.Cu") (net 7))
 (segment (start 129.7432 25.2984) (end 132.3086 22.733) (width 0.6096) (layer "B.Cu") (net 7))
 (segment (start 150.495 75.9841) (end 154.9908 80.4799) (width 0.6096) (layer "B.Cu") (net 7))
 (segment (start 91.8718 77.2287) (end 91.8718 75.1967) (width 0.6096) (layer "B.Cu") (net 7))
 (segment (start 129.7432 37.9839) (end 129.7432 25.2984) (width 0.6096) (layer "B.Cu") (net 7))
 (segment (start 140.3858 105.4481) (end 140.3858 134.9375) (width 0.6096) (layer "B.Cu") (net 7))
 (segment (start 132.2082 40.4489) (end 132.2082 47.6135) (width 0.6096) (layer "B.Cu") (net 7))
 (segment (start 78.0542 78.1939) (end 90.9066 78.1939) (width 0.6096) (layer "B.Cu") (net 7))
 (segment (start 73.914 129.4765) (end 73.914 82.3341) (width 0.6096) (layer "B.Cu") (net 7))
 (segment (start 86.7918 75.1967) (end 86.7918 73.2663) (width 0.6096) (layer "B.Cu") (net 4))
 (segment (start 86.0552 52.2859) (end 84.3534 50.5841) (width 0.6096) (layer "B.Cu") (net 4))
 (segment (start 101.346 26.3271) (end 103.3526 26.3271) (width 0.6096) (layer "B.Cu") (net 4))
 (segment (start 150.3882 40.4489) (end 146.0246 36.0853) (width 0.6096) (layer "B.Cu") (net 4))
 (segment (start 81.4832 26.7843) (end 84.4296 29.7307) (width 0.6096) (layer "B.Cu") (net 4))
 (segment (start 139.5902 30.5155) (end 138.4808 29.4061) (width 0.6096) (layer "B.Cu") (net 4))
 (segment (start 86.7918 57.7977) (end 86.0552 57.0611) (width 0.6096) (layer "B.Cu") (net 4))
 (segment (start 100.1268 21.0693) (end 93.7768 21.0693) (width 0.6096) (layer "B.Cu") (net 4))
 (segment (start 93.7768 21.0693) (end 84.201 21.0693) (width 0.6096) (layer "B.Cu") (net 4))
 (segment (start 86.7918 73.2663) (end 89.535 70.5231) (width 0.6096) (layer "B.Cu") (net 4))
 (segment (start 136.144 21.0693) (end 100.1268 21.0693) (width 0.6096) (layer "B.Cu") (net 4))
 (segment (start 86.0552 57.0611) (end 86.0552 52.2859) (width 0.6096) (layer "B.Cu") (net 4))
 (segment (start 81.4832 23.7871) (end 81.4832 26.7843) (width 0.6096) (layer "B.Cu") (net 4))
 (segment (start 146.0246 36.0853) (end 146.0246 31.7246) (width 0.6096) (layer "B.Cu") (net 4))
 (segment (start 89.535 70.5231) (end 89.535 63.8683) (width 0.6096) (layer "B.Cu") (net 4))
 (segment (start 84.201 21.0693) (end 81.4832 23.7871) (width 0.6096) (layer "B.Cu") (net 4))
 (segment (start 91.8464 23.4061) (end 93.7768 21.4757) (width 0.6096) (layer "B.Cu") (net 4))
 (segment (start 144.8155 30.5155) (end 139.5902 30.5155) (width 0.6096) (layer "B.Cu") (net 4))
 (segment (start 84.4296 29.7307) (end 84.4296 47.9933) (width 0.6096) (layer "B.Cu") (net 4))
 (segment (start 100.1268 21.0693) (end 100.1268 25.1079) (width 0.6096) (layer "B.Cu") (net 4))
 (segment (start 93.7768 21.4757) (end 93.7768 21.0693) (width 0.6096) (layer "B.Cu") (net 4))
 (segment (start 146.0246 31.7246) (end 144.8155 30.5155) (width 0.6096) (layer "B.Cu") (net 4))
 (segment (start 89.535 63.8683) (end 86.7918 61.1251) (width 0.6096) (layer "B.Cu") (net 4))
 (segment (start 138.4808 23.4061) (end 136.144 21.0693) (width 0.6096) (layer "B.Cu") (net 4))
 (segment (start 84.3534 48.0695) (end 84.4296 47.9933) (width 0.6096) (layer "B.Cu") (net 4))
 (segment (start 86.7918 61.1251) (end 86.7918 57.7977) (width 0.6096) (layer "B.Cu") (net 4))
 (segment (start 84.3534 50.5841) (end 84.3534 48.0695) (width 0.6096) (layer "B.Cu") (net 4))
 (segment (start 100.1268 25.1079) (end 101.346 26.3271) (width 0.6096) (layer "B.Cu") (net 4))
 (segment (start 97.917 40.8051) (end 97.917 31.0515) (width 0.4069) (layer "B.Cu") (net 48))
 (segment (start 100.1014 28.8671) (end 103.3526 28.8671) (width 0.4069) (layer "B.Cu") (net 48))
 (segment (start 97.917 31.0515) (end 100.1014 28.8671) (width 0.4069) (layer "B.Cu") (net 48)))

